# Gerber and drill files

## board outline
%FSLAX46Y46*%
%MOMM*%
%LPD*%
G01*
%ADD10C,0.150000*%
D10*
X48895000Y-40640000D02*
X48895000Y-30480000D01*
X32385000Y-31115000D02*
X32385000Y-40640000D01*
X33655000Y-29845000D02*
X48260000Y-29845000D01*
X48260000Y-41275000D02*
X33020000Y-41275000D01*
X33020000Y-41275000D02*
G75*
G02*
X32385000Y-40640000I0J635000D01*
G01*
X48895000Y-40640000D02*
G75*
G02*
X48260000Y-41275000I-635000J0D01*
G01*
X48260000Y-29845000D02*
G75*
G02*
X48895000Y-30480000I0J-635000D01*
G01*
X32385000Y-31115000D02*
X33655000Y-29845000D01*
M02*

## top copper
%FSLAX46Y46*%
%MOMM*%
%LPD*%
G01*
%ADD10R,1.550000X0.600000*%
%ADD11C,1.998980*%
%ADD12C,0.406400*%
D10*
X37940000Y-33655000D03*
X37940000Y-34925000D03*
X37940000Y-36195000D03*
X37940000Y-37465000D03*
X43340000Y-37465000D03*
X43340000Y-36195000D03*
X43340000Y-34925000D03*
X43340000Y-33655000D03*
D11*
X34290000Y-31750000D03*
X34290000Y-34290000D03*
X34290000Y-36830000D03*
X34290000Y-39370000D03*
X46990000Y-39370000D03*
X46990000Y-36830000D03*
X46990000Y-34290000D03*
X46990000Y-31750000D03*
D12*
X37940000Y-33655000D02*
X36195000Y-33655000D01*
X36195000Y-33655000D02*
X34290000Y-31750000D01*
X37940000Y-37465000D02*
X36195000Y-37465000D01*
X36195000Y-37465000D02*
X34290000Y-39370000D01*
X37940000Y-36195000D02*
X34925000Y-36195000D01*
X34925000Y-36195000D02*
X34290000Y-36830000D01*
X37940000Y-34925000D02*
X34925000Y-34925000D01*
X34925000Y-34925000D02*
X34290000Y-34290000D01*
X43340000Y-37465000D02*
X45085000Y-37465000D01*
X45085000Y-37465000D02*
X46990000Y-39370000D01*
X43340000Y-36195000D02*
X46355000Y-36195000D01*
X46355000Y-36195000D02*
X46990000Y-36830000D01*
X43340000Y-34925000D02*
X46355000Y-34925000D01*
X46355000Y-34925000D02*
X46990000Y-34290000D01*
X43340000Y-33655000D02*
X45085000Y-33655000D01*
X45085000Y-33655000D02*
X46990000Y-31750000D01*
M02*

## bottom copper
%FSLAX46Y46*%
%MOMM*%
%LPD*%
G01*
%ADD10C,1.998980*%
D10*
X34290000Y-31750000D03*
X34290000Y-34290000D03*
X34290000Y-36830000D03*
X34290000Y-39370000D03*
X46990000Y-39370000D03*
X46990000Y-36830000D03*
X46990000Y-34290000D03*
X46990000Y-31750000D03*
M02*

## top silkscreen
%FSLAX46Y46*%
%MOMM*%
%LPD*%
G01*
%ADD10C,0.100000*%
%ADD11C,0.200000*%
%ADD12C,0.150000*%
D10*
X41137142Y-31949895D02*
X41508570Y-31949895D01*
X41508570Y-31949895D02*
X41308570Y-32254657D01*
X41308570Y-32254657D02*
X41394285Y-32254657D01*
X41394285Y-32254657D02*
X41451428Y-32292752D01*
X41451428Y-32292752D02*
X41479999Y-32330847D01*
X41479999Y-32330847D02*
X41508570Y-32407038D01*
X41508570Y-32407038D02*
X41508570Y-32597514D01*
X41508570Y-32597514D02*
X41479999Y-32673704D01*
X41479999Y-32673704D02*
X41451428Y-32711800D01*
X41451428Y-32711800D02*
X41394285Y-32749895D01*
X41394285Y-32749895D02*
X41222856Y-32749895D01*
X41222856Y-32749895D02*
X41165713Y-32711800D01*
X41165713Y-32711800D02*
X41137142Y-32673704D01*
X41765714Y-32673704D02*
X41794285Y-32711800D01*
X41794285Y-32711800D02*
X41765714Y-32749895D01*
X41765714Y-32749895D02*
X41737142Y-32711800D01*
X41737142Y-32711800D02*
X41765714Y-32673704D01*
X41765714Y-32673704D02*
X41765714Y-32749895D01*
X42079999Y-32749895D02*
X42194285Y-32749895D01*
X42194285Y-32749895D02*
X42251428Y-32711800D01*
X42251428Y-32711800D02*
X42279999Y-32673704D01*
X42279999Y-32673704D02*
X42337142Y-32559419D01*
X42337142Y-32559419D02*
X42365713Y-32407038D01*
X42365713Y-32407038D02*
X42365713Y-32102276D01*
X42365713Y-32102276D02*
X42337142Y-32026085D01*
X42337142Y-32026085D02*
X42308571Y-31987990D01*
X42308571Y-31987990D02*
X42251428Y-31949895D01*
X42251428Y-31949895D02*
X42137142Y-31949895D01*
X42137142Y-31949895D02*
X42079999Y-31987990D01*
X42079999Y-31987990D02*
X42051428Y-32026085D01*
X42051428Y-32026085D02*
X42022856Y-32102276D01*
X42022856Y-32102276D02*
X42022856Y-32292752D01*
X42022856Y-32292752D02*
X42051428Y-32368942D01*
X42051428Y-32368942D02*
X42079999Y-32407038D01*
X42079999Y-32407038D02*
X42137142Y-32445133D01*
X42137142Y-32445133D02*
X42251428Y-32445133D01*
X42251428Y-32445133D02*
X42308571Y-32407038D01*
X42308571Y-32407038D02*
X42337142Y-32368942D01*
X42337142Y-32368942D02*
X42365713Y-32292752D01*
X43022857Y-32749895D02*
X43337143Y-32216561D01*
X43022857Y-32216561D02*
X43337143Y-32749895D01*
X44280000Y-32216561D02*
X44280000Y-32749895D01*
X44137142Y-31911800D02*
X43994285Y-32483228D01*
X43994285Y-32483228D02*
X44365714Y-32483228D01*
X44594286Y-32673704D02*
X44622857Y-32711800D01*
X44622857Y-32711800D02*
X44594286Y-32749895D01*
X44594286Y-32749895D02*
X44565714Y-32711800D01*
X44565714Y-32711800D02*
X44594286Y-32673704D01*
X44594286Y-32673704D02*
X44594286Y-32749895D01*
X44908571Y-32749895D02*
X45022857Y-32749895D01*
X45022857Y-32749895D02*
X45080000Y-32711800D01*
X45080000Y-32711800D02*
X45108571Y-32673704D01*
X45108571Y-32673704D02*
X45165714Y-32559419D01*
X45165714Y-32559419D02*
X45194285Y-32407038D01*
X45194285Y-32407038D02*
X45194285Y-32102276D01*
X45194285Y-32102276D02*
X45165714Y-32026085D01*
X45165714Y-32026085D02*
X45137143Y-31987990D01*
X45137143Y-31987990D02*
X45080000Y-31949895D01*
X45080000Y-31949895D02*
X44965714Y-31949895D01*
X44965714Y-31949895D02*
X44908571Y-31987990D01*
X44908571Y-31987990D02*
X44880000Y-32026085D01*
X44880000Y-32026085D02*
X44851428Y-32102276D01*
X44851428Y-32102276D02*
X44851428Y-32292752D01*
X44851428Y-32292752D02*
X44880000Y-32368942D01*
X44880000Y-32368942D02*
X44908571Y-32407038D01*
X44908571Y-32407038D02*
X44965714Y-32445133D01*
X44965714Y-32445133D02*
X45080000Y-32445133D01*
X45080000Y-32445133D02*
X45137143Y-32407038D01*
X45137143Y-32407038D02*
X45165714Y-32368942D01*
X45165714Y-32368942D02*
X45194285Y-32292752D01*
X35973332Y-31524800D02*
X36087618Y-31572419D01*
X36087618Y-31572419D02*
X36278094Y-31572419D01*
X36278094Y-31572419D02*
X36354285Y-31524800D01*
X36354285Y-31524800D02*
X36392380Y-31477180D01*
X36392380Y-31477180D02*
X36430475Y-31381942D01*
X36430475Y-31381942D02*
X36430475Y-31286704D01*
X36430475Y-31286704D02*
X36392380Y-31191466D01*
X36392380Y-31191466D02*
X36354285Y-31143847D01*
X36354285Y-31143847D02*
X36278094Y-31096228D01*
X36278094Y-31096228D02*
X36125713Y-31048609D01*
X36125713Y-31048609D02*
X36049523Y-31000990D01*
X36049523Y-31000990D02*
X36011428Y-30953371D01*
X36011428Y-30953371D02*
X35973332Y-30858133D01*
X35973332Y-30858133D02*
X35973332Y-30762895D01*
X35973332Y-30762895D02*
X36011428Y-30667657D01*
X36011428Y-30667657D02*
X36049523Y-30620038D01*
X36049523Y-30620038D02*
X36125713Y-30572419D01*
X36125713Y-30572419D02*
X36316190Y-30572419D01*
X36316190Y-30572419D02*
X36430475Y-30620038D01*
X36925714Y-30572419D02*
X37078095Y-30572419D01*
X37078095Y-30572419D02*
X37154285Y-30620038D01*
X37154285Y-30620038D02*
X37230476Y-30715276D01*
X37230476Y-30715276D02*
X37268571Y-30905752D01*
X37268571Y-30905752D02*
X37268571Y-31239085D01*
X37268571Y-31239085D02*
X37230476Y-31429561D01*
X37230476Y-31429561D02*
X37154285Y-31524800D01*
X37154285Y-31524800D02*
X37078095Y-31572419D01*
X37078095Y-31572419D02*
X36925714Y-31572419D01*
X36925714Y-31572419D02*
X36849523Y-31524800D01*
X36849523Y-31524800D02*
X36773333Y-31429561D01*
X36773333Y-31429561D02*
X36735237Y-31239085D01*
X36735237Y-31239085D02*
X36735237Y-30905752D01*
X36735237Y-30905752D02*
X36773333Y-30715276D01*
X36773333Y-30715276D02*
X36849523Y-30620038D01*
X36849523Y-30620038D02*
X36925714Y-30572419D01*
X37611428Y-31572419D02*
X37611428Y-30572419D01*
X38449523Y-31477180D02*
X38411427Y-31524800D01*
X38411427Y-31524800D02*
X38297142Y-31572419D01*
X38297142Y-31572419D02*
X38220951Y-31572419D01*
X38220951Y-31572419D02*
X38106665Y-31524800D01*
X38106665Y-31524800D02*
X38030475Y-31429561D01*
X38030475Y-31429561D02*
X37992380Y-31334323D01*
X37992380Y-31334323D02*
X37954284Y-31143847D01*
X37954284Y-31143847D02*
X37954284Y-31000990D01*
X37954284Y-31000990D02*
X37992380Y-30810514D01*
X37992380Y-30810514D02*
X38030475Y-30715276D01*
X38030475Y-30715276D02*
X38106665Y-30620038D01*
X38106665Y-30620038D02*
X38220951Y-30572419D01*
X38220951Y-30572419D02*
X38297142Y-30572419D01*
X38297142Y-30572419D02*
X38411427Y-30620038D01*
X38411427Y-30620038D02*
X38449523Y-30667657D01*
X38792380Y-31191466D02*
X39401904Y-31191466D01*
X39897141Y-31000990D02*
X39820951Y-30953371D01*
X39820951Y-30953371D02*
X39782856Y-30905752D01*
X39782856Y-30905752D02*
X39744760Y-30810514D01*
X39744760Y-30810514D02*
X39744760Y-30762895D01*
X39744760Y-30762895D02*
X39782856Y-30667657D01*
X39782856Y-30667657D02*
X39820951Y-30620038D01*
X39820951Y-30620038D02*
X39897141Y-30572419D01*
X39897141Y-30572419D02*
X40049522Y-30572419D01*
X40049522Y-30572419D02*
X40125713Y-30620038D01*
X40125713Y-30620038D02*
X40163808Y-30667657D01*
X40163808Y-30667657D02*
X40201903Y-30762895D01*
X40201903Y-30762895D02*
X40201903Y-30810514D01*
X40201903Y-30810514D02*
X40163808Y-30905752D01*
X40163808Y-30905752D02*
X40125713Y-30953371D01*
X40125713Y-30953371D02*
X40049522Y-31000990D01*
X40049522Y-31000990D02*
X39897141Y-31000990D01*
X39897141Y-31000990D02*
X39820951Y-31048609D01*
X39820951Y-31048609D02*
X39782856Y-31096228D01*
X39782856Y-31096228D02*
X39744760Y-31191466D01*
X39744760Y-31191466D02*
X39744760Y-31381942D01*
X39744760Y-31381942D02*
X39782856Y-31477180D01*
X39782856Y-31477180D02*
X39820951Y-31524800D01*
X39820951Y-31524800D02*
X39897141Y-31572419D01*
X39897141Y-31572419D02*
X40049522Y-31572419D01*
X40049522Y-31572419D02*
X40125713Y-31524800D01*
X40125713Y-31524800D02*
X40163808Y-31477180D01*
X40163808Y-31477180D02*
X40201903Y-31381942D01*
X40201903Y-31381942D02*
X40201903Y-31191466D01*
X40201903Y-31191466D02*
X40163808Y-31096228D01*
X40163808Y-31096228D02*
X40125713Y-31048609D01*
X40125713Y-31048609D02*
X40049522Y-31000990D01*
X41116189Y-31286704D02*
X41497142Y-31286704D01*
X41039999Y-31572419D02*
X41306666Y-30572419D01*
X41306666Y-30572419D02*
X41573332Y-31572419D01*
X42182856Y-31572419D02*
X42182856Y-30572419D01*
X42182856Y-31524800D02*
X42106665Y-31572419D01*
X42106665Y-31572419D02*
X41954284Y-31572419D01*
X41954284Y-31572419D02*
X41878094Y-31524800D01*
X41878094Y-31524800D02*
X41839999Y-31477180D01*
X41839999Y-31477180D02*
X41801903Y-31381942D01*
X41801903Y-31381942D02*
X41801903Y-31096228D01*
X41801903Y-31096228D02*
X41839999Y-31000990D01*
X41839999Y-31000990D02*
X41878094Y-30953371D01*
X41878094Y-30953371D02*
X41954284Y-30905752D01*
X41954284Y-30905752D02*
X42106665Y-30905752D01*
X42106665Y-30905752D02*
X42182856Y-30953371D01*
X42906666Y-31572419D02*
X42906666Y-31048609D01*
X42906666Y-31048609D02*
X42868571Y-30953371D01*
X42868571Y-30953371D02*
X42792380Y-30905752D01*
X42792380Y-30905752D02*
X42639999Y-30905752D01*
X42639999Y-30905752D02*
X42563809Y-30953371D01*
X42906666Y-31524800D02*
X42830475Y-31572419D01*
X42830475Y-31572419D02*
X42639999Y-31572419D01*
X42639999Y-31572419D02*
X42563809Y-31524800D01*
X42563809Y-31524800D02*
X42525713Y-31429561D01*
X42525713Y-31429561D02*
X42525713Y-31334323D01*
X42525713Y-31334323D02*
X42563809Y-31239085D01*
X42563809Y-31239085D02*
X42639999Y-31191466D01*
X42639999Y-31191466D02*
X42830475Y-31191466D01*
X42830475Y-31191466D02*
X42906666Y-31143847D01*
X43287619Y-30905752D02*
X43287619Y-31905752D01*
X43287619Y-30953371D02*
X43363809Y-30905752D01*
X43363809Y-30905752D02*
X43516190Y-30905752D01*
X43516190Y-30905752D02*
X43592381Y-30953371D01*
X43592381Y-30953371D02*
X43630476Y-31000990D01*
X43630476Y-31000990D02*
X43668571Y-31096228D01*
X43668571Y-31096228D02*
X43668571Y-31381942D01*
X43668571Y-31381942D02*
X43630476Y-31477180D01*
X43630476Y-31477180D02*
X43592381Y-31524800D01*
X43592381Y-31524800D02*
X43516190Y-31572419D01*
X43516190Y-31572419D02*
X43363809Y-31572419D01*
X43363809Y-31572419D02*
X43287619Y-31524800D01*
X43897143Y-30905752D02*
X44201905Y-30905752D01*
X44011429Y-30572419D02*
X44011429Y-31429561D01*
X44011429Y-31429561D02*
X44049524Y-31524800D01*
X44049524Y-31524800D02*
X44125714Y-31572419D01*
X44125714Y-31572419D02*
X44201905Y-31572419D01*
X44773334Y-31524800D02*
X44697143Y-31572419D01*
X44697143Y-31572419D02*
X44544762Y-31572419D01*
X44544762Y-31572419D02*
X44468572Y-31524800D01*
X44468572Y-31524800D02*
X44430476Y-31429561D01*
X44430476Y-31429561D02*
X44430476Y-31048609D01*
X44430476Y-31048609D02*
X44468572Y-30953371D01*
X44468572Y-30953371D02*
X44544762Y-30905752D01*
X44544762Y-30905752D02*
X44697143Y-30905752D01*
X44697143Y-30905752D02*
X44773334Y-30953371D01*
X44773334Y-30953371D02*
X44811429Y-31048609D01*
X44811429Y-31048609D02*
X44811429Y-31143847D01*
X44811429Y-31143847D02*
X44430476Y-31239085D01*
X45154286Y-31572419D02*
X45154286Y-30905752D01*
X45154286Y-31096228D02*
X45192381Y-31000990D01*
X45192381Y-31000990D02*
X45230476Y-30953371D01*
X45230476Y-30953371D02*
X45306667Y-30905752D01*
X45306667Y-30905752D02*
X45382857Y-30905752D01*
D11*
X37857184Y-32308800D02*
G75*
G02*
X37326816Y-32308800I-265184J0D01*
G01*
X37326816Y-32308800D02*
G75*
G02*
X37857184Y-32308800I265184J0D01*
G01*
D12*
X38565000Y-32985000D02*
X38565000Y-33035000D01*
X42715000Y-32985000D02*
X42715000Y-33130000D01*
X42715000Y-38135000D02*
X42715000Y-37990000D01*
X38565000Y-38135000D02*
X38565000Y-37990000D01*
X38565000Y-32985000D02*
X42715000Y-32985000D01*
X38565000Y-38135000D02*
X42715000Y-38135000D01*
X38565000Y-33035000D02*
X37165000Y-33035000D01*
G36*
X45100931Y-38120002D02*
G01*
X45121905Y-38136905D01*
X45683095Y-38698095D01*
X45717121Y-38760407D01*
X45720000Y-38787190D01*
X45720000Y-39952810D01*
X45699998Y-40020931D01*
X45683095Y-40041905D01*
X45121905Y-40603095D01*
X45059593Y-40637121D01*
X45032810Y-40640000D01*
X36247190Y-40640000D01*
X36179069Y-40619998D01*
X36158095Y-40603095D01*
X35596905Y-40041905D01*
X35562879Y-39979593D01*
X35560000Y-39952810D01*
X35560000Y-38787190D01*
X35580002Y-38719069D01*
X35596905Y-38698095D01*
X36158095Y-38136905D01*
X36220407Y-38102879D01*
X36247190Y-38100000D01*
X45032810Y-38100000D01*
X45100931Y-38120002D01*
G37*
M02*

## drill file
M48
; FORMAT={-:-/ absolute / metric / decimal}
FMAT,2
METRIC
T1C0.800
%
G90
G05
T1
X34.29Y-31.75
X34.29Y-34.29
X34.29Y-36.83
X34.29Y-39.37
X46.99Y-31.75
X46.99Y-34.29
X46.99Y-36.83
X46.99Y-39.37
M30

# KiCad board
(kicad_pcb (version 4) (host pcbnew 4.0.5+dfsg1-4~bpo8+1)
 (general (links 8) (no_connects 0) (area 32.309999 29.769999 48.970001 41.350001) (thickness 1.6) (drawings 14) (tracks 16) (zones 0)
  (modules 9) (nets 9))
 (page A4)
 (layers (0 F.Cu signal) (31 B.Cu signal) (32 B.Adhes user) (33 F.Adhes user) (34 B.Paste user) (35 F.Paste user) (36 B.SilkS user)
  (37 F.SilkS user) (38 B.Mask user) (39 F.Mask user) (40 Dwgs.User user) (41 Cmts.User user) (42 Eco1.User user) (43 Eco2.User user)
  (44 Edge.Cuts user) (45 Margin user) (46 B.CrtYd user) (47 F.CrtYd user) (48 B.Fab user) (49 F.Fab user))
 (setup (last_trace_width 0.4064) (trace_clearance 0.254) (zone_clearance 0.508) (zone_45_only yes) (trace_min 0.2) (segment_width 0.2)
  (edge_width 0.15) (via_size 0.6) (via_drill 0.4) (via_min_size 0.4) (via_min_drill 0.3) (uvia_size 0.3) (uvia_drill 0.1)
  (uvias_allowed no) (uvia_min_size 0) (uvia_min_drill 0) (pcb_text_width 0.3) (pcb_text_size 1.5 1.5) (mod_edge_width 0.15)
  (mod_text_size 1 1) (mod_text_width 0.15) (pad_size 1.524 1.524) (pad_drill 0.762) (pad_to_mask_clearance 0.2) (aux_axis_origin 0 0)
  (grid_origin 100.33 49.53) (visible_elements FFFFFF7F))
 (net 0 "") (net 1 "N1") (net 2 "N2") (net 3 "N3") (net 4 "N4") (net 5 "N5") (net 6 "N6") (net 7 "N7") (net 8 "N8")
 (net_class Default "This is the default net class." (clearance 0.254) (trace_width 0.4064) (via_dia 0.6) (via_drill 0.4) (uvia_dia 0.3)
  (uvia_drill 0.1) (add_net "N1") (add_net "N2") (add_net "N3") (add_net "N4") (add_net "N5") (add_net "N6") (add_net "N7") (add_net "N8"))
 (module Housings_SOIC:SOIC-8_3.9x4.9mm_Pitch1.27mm (layer F.Cu) (at 40.64 35.56)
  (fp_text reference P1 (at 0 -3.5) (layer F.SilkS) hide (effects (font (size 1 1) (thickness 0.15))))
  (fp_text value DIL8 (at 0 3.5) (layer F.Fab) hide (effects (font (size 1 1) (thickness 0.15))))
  (fp_line (start -2.075 -2.575) (end -2.075 -2.525) (layer F.SilkS) (width 0.15))
  (fp_line (start 2.075 -2.575) (end 2.075 -2.43) (layer F.SilkS) (width 0.15))
  (fp_line (start 2.075 2.575) (end 2.075 2.43) (layer F.SilkS) (width 0.15))
  (fp_line (start -2.075 2.575) (end -2.075 2.43) (layer F.SilkS) (width 0.15))
  (fp_line (start -2.075 -2.575) (end 2.075 -2.575) (layer F.SilkS) (width 0.15))
  (fp_line (start -2.075 2.575) (end 2.075 2.575) (layer F.SilkS) (width 0.15))
  (fp_line (start -2.075 -2.525) (end -3.475 -2.525) (layer F.SilkS) (width 0.15))
  (pad 1 smd rect (at -2.7 -1.905) (size 1.55 0.6) (layers F.Cu F.Paste F.Mask) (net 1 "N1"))
  (pad 2 smd rect (at -2.7 -0.635) (size 1.55 0.6) (layers F.Cu F.Paste F.Mask) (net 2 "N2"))
  (pad 3 smd rect (at -2.7 0.635) (size 1.55 0.6) (layers F.Cu F.Paste F.Mask) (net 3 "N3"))
  (pad 4 smd rect (at -2.7 1.905) (size 1.55 0.6) (layers F.Cu F.Paste F.Mask) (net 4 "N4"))
  (pad 5 smd rect (at 2.7 1.905) (size 1.55 0.6) (layers F.Cu F.Paste F.Mask) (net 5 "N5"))
  (pad 6 smd rect (at 2.7 0.635) (size 1.55 0.6) (layers F.Cu F.Paste F.Mask) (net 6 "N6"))
  (pad 7 smd rect (at 2.7 -0.635) (size 1.55 0.6) (layers F.Cu F.Paste F.Mask) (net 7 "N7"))
  (pad 8 smd rect (at 2.7 -1.905) (size 1.55 0.6) (layers F.Cu F.Paste F.Mask) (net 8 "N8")))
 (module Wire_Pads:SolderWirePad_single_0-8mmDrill (layer F.Cu) (at 34.29 31.75)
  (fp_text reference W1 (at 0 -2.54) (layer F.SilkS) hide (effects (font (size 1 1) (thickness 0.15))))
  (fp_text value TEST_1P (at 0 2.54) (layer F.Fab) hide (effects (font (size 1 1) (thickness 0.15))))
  (pad 1 thru_hole circle (at 0 0) (size 1.99898 1.99898) (drill 0.8001) (layers *.Cu *.Mask) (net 1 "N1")))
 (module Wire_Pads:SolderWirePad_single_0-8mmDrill (layer F.Cu) (at 34.29 34.29)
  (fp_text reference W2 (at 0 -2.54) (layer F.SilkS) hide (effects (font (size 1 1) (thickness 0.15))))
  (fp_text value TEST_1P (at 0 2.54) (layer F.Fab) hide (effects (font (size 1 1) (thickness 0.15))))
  (pad 1 thru_hole circle (at 0 0) (size 1.99898 1.99898) (drill 0.8001) (layers *.Cu *.Mask) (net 2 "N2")))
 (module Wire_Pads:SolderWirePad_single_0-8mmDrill (layer F.Cu) (at 34.29 36.83)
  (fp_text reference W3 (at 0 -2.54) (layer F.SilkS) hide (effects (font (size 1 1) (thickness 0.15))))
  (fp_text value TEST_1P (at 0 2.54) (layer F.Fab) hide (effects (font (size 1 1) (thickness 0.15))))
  (pad 1 thru_hole circle (at 0 0) (size 1.99898 1.99898) (drill 0.8001) (layers *.Cu *.Mask) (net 3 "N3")))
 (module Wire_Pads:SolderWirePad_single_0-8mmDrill (layer F.Cu) (at 34.29 39.37)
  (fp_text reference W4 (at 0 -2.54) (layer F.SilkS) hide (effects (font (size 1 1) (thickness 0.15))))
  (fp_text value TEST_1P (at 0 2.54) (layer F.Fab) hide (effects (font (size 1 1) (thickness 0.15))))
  (pad 1 thru_hole circle (at 0 0) (size 1.99898 1.99898) (drill 0.8001) (layers *.Cu *.Mask) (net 4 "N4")))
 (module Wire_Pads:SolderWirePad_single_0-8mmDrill (layer F.Cu) (at 46.99 39.37)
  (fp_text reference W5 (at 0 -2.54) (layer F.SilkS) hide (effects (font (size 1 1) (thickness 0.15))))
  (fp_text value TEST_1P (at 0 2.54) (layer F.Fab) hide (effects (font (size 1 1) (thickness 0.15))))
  (pad 1 thru_hole circle (at 0 0) (size 1.99898 1.99898) (drill 0.8001) (layers *.Cu *.Mask) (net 5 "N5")))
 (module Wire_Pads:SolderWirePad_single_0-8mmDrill (layer F.Cu) (at 46.99 36.83)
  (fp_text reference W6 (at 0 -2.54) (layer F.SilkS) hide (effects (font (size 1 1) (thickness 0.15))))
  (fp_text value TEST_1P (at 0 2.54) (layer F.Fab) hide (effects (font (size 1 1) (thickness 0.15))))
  (pad 1 thru_hole circle (at 0 0) (size 1.99898 1.99898) (drill 0.8001) (layers *.Cu *.Mask) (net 6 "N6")))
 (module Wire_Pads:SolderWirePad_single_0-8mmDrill (layer F.Cu) (at 46.99 34.29)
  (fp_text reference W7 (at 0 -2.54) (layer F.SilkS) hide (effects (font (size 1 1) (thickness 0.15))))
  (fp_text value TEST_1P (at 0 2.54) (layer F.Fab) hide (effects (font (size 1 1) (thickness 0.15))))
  (pad 1 thru_hole circle (at 0 0) (size 1.99898 1.99898) (drill 0.8001) (layers *.Cu *.Mask) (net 7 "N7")))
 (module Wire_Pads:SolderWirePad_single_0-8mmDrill (layer F.Cu) (at 46.99 31.75)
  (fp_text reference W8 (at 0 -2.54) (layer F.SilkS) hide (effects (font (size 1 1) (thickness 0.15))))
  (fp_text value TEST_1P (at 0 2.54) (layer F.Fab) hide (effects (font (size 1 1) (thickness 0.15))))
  (pad 1 thru_hole circle (at 0 0) (size 1.99898 1.99898) (drill 0.8001) (layers *.Cu *.Mask) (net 8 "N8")))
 (gr_line (start 48.895 40.64) (end 48.895 30.48) (angle 90) (layer Edge.Cuts) (width 0.15))
 (gr_line (start 32.385 31.115) (end 32.385 40.64) (angle 90) (layer Edge.Cuts) (width 0.15))
 (gr_line (start 33.655 29.845) (end 48.26 29.845) (angle 90) (layer Edge.Cuts) (width 0.15))
 (gr_line (start 48.26 41.275) (end 33.02 41.275) (angle 90) (layer Edge.Cuts) (width 0.15))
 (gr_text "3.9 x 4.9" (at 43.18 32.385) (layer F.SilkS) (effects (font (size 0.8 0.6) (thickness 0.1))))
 (gr_arc (start 33.02 40.64) (end 33.02 41.275) (angle 90) (layer Edge.Cuts) (width 0.15))
 (gr_arc (start 48.26 40.64) (end 48.895 40.64) (angle 90) (layer Edge.Cuts) (width 0.15))
 (gr_arc (start 48.26 30.48) (end 48.26 29.845) (angle 90) (layer Edge.Cuts) (width 0.15))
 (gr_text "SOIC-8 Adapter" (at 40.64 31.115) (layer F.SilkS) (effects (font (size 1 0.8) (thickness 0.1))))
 (gr_line (start 32.385 31.115) (end 33.655 29.845) (angle 90) (layer Edge.Cuts) (width 0.15))
 (gr_circle (center 37.592 32.3088) (end 37.338 32.2326) (layer F.SilkS) (width 0.2))
 (segment (start 37.94 33.655) (end 36.195 33.655) (width 0.4064) (layer F.Cu) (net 1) (status 400000))
 (segment (start 36.195 33.655) (end 34.29 31.75) (width 0.4064) (layer F.Cu) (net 1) (status 800000))
 (segment (start 37.94 37.465) (end 36.195 37.465) (width 0.4064) (layer F.Cu) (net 4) (status 400000))
 (segment (start 36.195 37.465) (end 34.29 39.37) (width 0.4064) (layer F.Cu) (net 4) (status 800000))
 (segment (start 37.94 36.195) (end 34.925 36.195) (width 0.4064) (layer F.Cu) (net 3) (status C00000))
 (segment (start 34.925 36.195) (end 34.29 36.83) (width 0.4064) (layer F.Cu) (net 3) (status C00000))
 (segment (start 37.94 34.925) (end 34.925 34.925) (width 0.4064) (layer F.Cu) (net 2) (status C00000))
 (segment (start 34.925 34.925) (end 34.29 34.29) (width 0.4064) (layer F.Cu) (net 2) (status C00000))
 (segment (start 43.34 37.465) (end 45.085 37.465) (width 0.4064) (layer F.Cu) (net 5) (status 400000))
 (segment (start 45.085 37.465) (end 46.99 39.37) (width 0.4064) (layer F.Cu) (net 5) (status 800000))
 (segment (start 43.34 36.195) (end 46.355 36.195) (width 0.4064) (layer F.Cu) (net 6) (status C00000))
 (segment (start 46.355 36.195) (end 46.99 36.83) (width 0.4064) (layer F.Cu) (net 6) (status C00000))
 (segment (start 43.34 34.925) (end 46.355 34.925) (width 0.4064) (layer F.Cu) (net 7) (status C00000))
 (segment (start 46.355 34.925) (end 46.99 34.29) (width 0.4064) (layer F.Cu) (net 7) (status C00000))
 (segment (start 43.34 33.655) (end 45.085 33.655) (width 0.4064) (layer F.Cu) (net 8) (status 400000))
 (segment (start 45.085 33.655) (end 46.99 31.75) (width 0.4064) (layer F.Cu) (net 8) (status 800000))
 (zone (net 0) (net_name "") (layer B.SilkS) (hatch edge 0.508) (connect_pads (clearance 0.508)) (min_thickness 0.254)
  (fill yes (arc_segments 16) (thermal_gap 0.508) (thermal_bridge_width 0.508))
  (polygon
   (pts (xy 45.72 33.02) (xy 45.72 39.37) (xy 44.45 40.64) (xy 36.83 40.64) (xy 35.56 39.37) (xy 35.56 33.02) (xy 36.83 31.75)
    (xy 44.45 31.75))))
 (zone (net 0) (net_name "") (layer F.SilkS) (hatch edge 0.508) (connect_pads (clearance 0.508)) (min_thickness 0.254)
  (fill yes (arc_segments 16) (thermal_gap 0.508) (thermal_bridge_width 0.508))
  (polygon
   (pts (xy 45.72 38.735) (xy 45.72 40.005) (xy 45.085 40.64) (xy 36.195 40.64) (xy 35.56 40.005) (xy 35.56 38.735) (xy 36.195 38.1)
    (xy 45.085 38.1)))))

